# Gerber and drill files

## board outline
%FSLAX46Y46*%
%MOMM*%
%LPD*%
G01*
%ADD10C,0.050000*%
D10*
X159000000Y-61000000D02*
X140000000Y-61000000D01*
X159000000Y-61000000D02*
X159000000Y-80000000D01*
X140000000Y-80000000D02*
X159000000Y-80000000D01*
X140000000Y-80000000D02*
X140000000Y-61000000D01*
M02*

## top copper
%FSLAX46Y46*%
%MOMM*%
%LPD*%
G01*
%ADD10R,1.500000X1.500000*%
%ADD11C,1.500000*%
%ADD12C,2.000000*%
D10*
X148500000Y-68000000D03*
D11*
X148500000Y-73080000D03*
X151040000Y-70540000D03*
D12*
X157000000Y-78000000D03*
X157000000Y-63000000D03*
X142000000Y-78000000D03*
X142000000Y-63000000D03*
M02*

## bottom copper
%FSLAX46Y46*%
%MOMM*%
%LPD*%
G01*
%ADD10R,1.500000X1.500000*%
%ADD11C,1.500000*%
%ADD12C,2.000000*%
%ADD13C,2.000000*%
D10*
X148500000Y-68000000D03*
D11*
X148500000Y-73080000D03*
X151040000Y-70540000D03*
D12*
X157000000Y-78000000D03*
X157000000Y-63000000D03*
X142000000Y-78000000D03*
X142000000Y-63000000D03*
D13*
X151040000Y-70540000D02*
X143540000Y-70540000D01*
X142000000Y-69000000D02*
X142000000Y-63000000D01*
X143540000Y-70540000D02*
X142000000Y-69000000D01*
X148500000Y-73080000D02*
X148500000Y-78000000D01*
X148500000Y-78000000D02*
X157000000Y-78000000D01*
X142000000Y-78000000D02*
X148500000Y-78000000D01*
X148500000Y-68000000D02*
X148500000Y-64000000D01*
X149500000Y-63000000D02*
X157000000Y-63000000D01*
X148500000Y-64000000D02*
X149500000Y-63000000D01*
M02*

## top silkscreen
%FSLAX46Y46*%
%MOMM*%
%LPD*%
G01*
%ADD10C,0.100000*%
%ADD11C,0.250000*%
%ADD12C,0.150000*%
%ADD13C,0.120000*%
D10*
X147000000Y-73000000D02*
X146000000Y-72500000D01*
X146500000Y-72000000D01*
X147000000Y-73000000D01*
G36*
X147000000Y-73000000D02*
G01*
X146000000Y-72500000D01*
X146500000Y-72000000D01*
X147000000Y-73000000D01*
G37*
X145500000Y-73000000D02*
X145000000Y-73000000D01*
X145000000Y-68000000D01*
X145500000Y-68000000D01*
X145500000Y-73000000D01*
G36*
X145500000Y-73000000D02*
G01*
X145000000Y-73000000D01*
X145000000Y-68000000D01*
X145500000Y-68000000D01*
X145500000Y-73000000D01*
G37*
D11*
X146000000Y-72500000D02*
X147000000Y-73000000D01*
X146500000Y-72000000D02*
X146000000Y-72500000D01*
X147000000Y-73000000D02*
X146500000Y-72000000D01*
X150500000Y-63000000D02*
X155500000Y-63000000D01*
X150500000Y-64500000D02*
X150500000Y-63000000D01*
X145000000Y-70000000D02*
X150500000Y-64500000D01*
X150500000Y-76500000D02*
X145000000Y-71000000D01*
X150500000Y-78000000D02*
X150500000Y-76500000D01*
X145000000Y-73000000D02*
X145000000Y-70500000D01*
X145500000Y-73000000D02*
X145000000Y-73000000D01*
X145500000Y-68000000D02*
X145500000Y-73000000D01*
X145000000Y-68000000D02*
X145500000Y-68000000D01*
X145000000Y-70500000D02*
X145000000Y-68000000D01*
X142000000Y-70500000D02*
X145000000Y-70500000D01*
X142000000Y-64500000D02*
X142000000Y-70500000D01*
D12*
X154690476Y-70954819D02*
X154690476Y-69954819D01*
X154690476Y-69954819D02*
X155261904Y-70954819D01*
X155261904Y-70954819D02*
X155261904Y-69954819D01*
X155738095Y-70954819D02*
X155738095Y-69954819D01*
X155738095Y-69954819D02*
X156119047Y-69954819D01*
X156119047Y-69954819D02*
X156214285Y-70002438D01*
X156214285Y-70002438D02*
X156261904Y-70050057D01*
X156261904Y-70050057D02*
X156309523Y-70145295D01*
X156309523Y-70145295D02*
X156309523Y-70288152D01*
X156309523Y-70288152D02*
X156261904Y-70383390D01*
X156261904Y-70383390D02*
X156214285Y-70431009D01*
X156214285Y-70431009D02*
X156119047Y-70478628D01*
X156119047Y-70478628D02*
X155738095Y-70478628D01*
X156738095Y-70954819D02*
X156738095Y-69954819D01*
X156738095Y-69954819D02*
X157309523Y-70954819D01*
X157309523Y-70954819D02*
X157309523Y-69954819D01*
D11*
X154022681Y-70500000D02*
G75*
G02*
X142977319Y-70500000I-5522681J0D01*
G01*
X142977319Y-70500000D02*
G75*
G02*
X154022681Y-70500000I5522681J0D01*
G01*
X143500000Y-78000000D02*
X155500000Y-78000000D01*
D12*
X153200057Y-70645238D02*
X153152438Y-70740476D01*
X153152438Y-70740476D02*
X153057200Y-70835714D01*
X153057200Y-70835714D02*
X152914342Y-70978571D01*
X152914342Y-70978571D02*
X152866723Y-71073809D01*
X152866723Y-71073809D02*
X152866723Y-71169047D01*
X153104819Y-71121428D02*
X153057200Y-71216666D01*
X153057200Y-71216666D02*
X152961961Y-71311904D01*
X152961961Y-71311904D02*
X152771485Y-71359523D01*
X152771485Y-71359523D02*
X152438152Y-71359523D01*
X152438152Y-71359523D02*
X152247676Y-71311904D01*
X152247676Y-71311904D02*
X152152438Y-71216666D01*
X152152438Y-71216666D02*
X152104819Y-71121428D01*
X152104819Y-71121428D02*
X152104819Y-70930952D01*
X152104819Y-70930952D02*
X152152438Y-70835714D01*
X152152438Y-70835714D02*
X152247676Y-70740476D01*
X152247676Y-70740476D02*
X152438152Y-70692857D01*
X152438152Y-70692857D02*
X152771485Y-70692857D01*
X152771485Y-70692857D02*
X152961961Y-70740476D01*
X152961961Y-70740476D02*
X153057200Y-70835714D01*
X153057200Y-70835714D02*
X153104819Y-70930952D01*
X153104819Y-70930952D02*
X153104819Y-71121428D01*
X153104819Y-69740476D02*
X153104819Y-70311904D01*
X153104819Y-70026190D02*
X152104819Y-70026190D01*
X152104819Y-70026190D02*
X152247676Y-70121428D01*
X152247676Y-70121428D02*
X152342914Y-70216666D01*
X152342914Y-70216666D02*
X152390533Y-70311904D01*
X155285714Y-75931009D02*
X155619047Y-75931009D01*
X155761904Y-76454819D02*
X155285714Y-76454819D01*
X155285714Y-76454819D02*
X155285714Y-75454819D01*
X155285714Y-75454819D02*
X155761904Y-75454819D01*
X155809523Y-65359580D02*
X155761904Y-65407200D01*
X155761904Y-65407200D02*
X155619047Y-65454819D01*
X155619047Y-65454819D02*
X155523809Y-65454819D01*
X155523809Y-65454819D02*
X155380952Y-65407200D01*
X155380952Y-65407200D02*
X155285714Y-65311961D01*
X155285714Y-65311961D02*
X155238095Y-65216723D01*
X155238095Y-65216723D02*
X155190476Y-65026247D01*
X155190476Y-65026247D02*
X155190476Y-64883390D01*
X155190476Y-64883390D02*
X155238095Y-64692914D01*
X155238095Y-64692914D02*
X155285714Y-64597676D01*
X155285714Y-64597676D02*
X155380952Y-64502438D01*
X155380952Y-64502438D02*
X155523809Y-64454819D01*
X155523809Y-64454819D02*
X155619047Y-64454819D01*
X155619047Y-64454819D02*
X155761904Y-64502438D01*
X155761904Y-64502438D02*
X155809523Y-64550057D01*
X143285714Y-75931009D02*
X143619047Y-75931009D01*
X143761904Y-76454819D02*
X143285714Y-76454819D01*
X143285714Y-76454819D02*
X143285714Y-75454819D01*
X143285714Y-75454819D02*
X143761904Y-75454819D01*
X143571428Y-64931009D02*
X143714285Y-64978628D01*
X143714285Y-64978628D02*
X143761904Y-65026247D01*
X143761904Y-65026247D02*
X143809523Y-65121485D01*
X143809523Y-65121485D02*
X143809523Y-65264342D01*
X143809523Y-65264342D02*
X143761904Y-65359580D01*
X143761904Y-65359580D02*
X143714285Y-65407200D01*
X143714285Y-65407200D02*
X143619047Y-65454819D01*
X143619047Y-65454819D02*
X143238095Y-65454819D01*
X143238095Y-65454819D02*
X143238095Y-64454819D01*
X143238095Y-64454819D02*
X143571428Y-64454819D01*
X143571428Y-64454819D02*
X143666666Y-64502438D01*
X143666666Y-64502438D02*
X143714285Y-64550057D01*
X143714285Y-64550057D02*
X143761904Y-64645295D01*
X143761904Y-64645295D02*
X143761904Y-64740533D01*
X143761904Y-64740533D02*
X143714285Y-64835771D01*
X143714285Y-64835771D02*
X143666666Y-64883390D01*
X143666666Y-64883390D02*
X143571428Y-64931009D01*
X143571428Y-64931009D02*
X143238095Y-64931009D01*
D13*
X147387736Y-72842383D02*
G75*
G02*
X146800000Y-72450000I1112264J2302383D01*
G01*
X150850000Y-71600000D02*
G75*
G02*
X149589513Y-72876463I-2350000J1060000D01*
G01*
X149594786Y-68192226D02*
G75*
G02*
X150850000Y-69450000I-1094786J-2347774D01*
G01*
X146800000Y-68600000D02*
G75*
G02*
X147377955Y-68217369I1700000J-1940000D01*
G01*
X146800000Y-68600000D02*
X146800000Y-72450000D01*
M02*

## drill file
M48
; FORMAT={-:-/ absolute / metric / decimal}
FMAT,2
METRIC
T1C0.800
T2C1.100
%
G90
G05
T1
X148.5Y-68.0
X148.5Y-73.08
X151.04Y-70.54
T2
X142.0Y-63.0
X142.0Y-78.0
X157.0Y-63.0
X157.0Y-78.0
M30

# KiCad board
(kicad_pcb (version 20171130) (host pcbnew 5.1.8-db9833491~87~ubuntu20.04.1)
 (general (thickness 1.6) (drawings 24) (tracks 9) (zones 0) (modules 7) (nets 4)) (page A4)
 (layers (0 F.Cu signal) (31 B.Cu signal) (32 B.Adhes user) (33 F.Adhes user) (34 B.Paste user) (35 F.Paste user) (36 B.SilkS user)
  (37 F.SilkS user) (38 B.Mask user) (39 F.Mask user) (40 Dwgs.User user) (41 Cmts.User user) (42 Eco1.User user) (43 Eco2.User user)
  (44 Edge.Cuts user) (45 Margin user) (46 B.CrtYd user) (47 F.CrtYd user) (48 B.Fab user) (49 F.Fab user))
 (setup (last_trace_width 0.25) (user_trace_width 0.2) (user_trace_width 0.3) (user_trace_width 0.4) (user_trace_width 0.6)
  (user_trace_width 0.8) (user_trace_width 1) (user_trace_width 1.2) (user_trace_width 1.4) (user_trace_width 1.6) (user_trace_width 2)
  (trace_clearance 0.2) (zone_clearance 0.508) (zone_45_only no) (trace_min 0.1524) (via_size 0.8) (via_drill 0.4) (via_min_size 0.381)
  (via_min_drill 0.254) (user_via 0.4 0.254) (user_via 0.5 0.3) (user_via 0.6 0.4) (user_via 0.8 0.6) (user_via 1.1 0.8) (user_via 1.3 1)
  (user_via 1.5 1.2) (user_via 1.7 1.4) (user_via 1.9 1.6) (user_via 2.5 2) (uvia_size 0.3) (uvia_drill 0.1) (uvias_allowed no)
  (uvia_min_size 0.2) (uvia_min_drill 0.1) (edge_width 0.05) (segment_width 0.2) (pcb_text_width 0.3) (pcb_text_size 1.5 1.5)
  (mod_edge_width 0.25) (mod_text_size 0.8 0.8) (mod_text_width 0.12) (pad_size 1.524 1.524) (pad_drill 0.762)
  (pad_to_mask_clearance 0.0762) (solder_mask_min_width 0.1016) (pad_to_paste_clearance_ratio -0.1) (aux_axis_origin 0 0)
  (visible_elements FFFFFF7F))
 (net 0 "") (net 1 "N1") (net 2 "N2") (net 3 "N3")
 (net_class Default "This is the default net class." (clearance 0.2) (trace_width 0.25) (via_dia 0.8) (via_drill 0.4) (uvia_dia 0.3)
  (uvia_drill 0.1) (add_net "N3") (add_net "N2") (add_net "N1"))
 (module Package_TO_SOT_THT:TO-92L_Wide (layer F.Cu) (at 148.5 68 270)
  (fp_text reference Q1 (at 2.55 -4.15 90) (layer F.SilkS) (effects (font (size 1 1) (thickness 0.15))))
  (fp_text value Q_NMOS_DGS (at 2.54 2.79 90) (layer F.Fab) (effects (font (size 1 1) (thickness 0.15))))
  (fp_arc (start 2.54 0) (end 4.45 1.7) (angle -15.88591585) (layer F.SilkS) (width 0.12))
  (fp_arc (start 2.54 0) (end 3.6 -2.35) (angle 40.72153779) (layer F.SilkS) (width 0.12))
  (fp_arc (start 2.54 0) (end 1.45 -2.35) (angle -40.11670855) (layer F.SilkS) (width 0.12))
  (fp_arc (start 2.54 0) (end 0.6 1.7) (angle 15.44288892) (layer F.SilkS) (width 0.12))
  (fp_line (start 0.6 1.7) (end 4.45 1.7) (layer F.SilkS) (width 0.12))
  (pad 1 thru_hole rect (at 0 0 270) (size 1.5 1.5) (drill 0.8) (layers *.Cu *.Mask) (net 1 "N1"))
  (pad 3 thru_hole circle (at 5.08 0 270) (size 1.5 1.5) (drill 0.8) (layers *.Cu *.Mask) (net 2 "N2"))
  (pad 2 thru_hole circle (at 2.54 -2.54 270) (size 1.5 1.5) (drill 0.8) (layers *.Cu *.Mask) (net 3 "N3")))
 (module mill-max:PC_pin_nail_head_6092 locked (layer F.Cu) (at 157 78)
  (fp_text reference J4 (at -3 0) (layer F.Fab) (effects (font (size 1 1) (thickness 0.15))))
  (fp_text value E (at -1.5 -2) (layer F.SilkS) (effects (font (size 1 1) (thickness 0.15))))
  (pad 1 thru_hole circle (at 0 0) (size 2 2) (drill 1.1) (layers *.Cu *.Mask) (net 2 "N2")))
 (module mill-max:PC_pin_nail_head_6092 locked (layer F.Cu) (at 157 63)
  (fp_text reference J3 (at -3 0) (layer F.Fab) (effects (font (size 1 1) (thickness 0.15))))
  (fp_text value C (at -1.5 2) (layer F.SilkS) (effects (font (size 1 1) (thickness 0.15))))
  (pad 1 thru_hole circle (at 0 0) (size 2 2) (drill 1.1) (layers *.Cu *.Mask) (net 1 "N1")))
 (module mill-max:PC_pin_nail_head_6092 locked (layer F.Cu) (at 142 78)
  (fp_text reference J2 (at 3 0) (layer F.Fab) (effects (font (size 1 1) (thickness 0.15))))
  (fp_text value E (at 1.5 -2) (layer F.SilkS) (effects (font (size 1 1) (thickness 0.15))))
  (pad 1 thru_hole circle (at 0 0) (size 2 2) (drill 1.1) (layers *.Cu *.Mask) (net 2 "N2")))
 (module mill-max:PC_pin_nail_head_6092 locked (layer F.Cu) (at 142 63)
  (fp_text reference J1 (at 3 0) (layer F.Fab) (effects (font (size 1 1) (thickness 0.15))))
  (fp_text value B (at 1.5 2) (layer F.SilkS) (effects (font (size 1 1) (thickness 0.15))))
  (pad 1 thru_hole circle (at 0 0) (size 2 2) (drill 1.1) (layers *.Cu *.Mask) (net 3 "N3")))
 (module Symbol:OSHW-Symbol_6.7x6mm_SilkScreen (layer B.Cu) (at 155.5 70.5 270)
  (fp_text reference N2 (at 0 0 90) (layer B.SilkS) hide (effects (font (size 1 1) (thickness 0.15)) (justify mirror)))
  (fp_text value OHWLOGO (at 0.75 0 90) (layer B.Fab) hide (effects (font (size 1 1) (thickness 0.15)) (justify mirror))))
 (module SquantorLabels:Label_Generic (layer B.Cu) (at 141.5 71.5 90)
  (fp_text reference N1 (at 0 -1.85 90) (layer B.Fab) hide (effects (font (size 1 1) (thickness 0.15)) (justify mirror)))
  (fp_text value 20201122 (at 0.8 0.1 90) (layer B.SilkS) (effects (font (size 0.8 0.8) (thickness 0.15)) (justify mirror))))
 (gr_poly (pts (xy 147 73) (xy 146 72.5) (xy 146.5 72)) (layer F.SilkS) (width 0.1))
 (gr_poly (pts (xy 145.5 73) (xy 145 73) (xy 145 68) (xy 145.5 68)) (layer F.SilkS) (width 0.1))
 (gr_line (start 146 72.5) (end 147 73) (layer F.SilkS) (width 0.25))
 (gr_line (start 146.5 72) (end 146 72.5) (layer F.SilkS) (width 0.25))
 (gr_line (start 147 73) (end 146.5 72) (layer F.SilkS) (width 0.25))
 (gr_line (start 150.5 63) (end 155.5 63) (layer F.SilkS) (width 0.25))
 (gr_line (start 150.5 64.5) (end 150.5 63) (layer F.SilkS) (width 0.25))
 (gr_line (start 145 70) (end 150.5 64.5) (layer F.SilkS) (width 0.25))
 (gr_line (start 150.5 76.5) (end 145 71) (layer F.SilkS) (width 0.25))
 (gr_line (start 150.5 78) (end 150.5 76.5) (layer F.SilkS) (width 0.25))
 (gr_line (start 145 73) (end 145 70.5) (layer F.SilkS) (width 0.25))
 (gr_line (start 145.5 73) (end 145 73) (layer F.SilkS) (width 0.25))
 (gr_line (start 145.5 68) (end 145.5 73) (layer F.SilkS) (width 0.25))
 (gr_line (start 145 68) (end 145.5 68) (layer F.SilkS) (width 0.25))
 (gr_line (start 145 70.5) (end 145 68) (layer F.SilkS) (width 0.25))
 (gr_line (start 142 70.5) (end 145 70.5) (layer F.SilkS) (width 0.25))
 (gr_line (start 142 64.5) (end 142 70.5) (layer F.SilkS) (width 0.25))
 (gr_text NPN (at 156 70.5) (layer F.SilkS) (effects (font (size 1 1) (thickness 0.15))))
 (gr_circle (center 148.5 70.5) (end 154 71) (layer F.SilkS) (width 0.25))
 (gr_line (start 143.5 78) (end 155.5 78) (layer F.SilkS) (width 0.25))
 (gr_line (start 159 61) (end 140 61) (layer Edge.Cuts) (width 0.05))
 (gr_line (start 159 61) (end 159 80) (layer Edge.Cuts) (width 0.05))
 (gr_line (start 140 80) (end 159 80) (layer Edge.Cuts) (width 0.05))
 (gr_line (start 140 80) (end 140 61) (layer Edge.Cuts) (width 0.05))
 (segment (start 151.04 70.54) (end 143.54 70.54) (width 2) (layer B.Cu) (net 3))
 (segment (start 142 69) (end 142 63) (width 2) (layer B.Cu) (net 3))
 (segment (start 143.54 70.54) (end 142 69) (width 2) (layer B.Cu) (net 3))
 (segment (start 148.5 73.08) (end 148.5 78) (width 2) (layer B.Cu) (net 2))
 (segment (start 148.5 78) (end 157 78) (width 2) (layer B.Cu) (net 2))
 (segment (start 142 78) (end 148.5 78) (width 2) (layer B.Cu) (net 2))
 (segment (start 148.5 68) (end 148.5 64) (width 2) (layer B.Cu) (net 1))
 (segment (start 149.5 63) (end 157 63) (width 2) (layer B.Cu) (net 1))
 (segment (start 148.5 64) (end 149.5 63) (width 2) (layer B.Cu) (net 1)))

